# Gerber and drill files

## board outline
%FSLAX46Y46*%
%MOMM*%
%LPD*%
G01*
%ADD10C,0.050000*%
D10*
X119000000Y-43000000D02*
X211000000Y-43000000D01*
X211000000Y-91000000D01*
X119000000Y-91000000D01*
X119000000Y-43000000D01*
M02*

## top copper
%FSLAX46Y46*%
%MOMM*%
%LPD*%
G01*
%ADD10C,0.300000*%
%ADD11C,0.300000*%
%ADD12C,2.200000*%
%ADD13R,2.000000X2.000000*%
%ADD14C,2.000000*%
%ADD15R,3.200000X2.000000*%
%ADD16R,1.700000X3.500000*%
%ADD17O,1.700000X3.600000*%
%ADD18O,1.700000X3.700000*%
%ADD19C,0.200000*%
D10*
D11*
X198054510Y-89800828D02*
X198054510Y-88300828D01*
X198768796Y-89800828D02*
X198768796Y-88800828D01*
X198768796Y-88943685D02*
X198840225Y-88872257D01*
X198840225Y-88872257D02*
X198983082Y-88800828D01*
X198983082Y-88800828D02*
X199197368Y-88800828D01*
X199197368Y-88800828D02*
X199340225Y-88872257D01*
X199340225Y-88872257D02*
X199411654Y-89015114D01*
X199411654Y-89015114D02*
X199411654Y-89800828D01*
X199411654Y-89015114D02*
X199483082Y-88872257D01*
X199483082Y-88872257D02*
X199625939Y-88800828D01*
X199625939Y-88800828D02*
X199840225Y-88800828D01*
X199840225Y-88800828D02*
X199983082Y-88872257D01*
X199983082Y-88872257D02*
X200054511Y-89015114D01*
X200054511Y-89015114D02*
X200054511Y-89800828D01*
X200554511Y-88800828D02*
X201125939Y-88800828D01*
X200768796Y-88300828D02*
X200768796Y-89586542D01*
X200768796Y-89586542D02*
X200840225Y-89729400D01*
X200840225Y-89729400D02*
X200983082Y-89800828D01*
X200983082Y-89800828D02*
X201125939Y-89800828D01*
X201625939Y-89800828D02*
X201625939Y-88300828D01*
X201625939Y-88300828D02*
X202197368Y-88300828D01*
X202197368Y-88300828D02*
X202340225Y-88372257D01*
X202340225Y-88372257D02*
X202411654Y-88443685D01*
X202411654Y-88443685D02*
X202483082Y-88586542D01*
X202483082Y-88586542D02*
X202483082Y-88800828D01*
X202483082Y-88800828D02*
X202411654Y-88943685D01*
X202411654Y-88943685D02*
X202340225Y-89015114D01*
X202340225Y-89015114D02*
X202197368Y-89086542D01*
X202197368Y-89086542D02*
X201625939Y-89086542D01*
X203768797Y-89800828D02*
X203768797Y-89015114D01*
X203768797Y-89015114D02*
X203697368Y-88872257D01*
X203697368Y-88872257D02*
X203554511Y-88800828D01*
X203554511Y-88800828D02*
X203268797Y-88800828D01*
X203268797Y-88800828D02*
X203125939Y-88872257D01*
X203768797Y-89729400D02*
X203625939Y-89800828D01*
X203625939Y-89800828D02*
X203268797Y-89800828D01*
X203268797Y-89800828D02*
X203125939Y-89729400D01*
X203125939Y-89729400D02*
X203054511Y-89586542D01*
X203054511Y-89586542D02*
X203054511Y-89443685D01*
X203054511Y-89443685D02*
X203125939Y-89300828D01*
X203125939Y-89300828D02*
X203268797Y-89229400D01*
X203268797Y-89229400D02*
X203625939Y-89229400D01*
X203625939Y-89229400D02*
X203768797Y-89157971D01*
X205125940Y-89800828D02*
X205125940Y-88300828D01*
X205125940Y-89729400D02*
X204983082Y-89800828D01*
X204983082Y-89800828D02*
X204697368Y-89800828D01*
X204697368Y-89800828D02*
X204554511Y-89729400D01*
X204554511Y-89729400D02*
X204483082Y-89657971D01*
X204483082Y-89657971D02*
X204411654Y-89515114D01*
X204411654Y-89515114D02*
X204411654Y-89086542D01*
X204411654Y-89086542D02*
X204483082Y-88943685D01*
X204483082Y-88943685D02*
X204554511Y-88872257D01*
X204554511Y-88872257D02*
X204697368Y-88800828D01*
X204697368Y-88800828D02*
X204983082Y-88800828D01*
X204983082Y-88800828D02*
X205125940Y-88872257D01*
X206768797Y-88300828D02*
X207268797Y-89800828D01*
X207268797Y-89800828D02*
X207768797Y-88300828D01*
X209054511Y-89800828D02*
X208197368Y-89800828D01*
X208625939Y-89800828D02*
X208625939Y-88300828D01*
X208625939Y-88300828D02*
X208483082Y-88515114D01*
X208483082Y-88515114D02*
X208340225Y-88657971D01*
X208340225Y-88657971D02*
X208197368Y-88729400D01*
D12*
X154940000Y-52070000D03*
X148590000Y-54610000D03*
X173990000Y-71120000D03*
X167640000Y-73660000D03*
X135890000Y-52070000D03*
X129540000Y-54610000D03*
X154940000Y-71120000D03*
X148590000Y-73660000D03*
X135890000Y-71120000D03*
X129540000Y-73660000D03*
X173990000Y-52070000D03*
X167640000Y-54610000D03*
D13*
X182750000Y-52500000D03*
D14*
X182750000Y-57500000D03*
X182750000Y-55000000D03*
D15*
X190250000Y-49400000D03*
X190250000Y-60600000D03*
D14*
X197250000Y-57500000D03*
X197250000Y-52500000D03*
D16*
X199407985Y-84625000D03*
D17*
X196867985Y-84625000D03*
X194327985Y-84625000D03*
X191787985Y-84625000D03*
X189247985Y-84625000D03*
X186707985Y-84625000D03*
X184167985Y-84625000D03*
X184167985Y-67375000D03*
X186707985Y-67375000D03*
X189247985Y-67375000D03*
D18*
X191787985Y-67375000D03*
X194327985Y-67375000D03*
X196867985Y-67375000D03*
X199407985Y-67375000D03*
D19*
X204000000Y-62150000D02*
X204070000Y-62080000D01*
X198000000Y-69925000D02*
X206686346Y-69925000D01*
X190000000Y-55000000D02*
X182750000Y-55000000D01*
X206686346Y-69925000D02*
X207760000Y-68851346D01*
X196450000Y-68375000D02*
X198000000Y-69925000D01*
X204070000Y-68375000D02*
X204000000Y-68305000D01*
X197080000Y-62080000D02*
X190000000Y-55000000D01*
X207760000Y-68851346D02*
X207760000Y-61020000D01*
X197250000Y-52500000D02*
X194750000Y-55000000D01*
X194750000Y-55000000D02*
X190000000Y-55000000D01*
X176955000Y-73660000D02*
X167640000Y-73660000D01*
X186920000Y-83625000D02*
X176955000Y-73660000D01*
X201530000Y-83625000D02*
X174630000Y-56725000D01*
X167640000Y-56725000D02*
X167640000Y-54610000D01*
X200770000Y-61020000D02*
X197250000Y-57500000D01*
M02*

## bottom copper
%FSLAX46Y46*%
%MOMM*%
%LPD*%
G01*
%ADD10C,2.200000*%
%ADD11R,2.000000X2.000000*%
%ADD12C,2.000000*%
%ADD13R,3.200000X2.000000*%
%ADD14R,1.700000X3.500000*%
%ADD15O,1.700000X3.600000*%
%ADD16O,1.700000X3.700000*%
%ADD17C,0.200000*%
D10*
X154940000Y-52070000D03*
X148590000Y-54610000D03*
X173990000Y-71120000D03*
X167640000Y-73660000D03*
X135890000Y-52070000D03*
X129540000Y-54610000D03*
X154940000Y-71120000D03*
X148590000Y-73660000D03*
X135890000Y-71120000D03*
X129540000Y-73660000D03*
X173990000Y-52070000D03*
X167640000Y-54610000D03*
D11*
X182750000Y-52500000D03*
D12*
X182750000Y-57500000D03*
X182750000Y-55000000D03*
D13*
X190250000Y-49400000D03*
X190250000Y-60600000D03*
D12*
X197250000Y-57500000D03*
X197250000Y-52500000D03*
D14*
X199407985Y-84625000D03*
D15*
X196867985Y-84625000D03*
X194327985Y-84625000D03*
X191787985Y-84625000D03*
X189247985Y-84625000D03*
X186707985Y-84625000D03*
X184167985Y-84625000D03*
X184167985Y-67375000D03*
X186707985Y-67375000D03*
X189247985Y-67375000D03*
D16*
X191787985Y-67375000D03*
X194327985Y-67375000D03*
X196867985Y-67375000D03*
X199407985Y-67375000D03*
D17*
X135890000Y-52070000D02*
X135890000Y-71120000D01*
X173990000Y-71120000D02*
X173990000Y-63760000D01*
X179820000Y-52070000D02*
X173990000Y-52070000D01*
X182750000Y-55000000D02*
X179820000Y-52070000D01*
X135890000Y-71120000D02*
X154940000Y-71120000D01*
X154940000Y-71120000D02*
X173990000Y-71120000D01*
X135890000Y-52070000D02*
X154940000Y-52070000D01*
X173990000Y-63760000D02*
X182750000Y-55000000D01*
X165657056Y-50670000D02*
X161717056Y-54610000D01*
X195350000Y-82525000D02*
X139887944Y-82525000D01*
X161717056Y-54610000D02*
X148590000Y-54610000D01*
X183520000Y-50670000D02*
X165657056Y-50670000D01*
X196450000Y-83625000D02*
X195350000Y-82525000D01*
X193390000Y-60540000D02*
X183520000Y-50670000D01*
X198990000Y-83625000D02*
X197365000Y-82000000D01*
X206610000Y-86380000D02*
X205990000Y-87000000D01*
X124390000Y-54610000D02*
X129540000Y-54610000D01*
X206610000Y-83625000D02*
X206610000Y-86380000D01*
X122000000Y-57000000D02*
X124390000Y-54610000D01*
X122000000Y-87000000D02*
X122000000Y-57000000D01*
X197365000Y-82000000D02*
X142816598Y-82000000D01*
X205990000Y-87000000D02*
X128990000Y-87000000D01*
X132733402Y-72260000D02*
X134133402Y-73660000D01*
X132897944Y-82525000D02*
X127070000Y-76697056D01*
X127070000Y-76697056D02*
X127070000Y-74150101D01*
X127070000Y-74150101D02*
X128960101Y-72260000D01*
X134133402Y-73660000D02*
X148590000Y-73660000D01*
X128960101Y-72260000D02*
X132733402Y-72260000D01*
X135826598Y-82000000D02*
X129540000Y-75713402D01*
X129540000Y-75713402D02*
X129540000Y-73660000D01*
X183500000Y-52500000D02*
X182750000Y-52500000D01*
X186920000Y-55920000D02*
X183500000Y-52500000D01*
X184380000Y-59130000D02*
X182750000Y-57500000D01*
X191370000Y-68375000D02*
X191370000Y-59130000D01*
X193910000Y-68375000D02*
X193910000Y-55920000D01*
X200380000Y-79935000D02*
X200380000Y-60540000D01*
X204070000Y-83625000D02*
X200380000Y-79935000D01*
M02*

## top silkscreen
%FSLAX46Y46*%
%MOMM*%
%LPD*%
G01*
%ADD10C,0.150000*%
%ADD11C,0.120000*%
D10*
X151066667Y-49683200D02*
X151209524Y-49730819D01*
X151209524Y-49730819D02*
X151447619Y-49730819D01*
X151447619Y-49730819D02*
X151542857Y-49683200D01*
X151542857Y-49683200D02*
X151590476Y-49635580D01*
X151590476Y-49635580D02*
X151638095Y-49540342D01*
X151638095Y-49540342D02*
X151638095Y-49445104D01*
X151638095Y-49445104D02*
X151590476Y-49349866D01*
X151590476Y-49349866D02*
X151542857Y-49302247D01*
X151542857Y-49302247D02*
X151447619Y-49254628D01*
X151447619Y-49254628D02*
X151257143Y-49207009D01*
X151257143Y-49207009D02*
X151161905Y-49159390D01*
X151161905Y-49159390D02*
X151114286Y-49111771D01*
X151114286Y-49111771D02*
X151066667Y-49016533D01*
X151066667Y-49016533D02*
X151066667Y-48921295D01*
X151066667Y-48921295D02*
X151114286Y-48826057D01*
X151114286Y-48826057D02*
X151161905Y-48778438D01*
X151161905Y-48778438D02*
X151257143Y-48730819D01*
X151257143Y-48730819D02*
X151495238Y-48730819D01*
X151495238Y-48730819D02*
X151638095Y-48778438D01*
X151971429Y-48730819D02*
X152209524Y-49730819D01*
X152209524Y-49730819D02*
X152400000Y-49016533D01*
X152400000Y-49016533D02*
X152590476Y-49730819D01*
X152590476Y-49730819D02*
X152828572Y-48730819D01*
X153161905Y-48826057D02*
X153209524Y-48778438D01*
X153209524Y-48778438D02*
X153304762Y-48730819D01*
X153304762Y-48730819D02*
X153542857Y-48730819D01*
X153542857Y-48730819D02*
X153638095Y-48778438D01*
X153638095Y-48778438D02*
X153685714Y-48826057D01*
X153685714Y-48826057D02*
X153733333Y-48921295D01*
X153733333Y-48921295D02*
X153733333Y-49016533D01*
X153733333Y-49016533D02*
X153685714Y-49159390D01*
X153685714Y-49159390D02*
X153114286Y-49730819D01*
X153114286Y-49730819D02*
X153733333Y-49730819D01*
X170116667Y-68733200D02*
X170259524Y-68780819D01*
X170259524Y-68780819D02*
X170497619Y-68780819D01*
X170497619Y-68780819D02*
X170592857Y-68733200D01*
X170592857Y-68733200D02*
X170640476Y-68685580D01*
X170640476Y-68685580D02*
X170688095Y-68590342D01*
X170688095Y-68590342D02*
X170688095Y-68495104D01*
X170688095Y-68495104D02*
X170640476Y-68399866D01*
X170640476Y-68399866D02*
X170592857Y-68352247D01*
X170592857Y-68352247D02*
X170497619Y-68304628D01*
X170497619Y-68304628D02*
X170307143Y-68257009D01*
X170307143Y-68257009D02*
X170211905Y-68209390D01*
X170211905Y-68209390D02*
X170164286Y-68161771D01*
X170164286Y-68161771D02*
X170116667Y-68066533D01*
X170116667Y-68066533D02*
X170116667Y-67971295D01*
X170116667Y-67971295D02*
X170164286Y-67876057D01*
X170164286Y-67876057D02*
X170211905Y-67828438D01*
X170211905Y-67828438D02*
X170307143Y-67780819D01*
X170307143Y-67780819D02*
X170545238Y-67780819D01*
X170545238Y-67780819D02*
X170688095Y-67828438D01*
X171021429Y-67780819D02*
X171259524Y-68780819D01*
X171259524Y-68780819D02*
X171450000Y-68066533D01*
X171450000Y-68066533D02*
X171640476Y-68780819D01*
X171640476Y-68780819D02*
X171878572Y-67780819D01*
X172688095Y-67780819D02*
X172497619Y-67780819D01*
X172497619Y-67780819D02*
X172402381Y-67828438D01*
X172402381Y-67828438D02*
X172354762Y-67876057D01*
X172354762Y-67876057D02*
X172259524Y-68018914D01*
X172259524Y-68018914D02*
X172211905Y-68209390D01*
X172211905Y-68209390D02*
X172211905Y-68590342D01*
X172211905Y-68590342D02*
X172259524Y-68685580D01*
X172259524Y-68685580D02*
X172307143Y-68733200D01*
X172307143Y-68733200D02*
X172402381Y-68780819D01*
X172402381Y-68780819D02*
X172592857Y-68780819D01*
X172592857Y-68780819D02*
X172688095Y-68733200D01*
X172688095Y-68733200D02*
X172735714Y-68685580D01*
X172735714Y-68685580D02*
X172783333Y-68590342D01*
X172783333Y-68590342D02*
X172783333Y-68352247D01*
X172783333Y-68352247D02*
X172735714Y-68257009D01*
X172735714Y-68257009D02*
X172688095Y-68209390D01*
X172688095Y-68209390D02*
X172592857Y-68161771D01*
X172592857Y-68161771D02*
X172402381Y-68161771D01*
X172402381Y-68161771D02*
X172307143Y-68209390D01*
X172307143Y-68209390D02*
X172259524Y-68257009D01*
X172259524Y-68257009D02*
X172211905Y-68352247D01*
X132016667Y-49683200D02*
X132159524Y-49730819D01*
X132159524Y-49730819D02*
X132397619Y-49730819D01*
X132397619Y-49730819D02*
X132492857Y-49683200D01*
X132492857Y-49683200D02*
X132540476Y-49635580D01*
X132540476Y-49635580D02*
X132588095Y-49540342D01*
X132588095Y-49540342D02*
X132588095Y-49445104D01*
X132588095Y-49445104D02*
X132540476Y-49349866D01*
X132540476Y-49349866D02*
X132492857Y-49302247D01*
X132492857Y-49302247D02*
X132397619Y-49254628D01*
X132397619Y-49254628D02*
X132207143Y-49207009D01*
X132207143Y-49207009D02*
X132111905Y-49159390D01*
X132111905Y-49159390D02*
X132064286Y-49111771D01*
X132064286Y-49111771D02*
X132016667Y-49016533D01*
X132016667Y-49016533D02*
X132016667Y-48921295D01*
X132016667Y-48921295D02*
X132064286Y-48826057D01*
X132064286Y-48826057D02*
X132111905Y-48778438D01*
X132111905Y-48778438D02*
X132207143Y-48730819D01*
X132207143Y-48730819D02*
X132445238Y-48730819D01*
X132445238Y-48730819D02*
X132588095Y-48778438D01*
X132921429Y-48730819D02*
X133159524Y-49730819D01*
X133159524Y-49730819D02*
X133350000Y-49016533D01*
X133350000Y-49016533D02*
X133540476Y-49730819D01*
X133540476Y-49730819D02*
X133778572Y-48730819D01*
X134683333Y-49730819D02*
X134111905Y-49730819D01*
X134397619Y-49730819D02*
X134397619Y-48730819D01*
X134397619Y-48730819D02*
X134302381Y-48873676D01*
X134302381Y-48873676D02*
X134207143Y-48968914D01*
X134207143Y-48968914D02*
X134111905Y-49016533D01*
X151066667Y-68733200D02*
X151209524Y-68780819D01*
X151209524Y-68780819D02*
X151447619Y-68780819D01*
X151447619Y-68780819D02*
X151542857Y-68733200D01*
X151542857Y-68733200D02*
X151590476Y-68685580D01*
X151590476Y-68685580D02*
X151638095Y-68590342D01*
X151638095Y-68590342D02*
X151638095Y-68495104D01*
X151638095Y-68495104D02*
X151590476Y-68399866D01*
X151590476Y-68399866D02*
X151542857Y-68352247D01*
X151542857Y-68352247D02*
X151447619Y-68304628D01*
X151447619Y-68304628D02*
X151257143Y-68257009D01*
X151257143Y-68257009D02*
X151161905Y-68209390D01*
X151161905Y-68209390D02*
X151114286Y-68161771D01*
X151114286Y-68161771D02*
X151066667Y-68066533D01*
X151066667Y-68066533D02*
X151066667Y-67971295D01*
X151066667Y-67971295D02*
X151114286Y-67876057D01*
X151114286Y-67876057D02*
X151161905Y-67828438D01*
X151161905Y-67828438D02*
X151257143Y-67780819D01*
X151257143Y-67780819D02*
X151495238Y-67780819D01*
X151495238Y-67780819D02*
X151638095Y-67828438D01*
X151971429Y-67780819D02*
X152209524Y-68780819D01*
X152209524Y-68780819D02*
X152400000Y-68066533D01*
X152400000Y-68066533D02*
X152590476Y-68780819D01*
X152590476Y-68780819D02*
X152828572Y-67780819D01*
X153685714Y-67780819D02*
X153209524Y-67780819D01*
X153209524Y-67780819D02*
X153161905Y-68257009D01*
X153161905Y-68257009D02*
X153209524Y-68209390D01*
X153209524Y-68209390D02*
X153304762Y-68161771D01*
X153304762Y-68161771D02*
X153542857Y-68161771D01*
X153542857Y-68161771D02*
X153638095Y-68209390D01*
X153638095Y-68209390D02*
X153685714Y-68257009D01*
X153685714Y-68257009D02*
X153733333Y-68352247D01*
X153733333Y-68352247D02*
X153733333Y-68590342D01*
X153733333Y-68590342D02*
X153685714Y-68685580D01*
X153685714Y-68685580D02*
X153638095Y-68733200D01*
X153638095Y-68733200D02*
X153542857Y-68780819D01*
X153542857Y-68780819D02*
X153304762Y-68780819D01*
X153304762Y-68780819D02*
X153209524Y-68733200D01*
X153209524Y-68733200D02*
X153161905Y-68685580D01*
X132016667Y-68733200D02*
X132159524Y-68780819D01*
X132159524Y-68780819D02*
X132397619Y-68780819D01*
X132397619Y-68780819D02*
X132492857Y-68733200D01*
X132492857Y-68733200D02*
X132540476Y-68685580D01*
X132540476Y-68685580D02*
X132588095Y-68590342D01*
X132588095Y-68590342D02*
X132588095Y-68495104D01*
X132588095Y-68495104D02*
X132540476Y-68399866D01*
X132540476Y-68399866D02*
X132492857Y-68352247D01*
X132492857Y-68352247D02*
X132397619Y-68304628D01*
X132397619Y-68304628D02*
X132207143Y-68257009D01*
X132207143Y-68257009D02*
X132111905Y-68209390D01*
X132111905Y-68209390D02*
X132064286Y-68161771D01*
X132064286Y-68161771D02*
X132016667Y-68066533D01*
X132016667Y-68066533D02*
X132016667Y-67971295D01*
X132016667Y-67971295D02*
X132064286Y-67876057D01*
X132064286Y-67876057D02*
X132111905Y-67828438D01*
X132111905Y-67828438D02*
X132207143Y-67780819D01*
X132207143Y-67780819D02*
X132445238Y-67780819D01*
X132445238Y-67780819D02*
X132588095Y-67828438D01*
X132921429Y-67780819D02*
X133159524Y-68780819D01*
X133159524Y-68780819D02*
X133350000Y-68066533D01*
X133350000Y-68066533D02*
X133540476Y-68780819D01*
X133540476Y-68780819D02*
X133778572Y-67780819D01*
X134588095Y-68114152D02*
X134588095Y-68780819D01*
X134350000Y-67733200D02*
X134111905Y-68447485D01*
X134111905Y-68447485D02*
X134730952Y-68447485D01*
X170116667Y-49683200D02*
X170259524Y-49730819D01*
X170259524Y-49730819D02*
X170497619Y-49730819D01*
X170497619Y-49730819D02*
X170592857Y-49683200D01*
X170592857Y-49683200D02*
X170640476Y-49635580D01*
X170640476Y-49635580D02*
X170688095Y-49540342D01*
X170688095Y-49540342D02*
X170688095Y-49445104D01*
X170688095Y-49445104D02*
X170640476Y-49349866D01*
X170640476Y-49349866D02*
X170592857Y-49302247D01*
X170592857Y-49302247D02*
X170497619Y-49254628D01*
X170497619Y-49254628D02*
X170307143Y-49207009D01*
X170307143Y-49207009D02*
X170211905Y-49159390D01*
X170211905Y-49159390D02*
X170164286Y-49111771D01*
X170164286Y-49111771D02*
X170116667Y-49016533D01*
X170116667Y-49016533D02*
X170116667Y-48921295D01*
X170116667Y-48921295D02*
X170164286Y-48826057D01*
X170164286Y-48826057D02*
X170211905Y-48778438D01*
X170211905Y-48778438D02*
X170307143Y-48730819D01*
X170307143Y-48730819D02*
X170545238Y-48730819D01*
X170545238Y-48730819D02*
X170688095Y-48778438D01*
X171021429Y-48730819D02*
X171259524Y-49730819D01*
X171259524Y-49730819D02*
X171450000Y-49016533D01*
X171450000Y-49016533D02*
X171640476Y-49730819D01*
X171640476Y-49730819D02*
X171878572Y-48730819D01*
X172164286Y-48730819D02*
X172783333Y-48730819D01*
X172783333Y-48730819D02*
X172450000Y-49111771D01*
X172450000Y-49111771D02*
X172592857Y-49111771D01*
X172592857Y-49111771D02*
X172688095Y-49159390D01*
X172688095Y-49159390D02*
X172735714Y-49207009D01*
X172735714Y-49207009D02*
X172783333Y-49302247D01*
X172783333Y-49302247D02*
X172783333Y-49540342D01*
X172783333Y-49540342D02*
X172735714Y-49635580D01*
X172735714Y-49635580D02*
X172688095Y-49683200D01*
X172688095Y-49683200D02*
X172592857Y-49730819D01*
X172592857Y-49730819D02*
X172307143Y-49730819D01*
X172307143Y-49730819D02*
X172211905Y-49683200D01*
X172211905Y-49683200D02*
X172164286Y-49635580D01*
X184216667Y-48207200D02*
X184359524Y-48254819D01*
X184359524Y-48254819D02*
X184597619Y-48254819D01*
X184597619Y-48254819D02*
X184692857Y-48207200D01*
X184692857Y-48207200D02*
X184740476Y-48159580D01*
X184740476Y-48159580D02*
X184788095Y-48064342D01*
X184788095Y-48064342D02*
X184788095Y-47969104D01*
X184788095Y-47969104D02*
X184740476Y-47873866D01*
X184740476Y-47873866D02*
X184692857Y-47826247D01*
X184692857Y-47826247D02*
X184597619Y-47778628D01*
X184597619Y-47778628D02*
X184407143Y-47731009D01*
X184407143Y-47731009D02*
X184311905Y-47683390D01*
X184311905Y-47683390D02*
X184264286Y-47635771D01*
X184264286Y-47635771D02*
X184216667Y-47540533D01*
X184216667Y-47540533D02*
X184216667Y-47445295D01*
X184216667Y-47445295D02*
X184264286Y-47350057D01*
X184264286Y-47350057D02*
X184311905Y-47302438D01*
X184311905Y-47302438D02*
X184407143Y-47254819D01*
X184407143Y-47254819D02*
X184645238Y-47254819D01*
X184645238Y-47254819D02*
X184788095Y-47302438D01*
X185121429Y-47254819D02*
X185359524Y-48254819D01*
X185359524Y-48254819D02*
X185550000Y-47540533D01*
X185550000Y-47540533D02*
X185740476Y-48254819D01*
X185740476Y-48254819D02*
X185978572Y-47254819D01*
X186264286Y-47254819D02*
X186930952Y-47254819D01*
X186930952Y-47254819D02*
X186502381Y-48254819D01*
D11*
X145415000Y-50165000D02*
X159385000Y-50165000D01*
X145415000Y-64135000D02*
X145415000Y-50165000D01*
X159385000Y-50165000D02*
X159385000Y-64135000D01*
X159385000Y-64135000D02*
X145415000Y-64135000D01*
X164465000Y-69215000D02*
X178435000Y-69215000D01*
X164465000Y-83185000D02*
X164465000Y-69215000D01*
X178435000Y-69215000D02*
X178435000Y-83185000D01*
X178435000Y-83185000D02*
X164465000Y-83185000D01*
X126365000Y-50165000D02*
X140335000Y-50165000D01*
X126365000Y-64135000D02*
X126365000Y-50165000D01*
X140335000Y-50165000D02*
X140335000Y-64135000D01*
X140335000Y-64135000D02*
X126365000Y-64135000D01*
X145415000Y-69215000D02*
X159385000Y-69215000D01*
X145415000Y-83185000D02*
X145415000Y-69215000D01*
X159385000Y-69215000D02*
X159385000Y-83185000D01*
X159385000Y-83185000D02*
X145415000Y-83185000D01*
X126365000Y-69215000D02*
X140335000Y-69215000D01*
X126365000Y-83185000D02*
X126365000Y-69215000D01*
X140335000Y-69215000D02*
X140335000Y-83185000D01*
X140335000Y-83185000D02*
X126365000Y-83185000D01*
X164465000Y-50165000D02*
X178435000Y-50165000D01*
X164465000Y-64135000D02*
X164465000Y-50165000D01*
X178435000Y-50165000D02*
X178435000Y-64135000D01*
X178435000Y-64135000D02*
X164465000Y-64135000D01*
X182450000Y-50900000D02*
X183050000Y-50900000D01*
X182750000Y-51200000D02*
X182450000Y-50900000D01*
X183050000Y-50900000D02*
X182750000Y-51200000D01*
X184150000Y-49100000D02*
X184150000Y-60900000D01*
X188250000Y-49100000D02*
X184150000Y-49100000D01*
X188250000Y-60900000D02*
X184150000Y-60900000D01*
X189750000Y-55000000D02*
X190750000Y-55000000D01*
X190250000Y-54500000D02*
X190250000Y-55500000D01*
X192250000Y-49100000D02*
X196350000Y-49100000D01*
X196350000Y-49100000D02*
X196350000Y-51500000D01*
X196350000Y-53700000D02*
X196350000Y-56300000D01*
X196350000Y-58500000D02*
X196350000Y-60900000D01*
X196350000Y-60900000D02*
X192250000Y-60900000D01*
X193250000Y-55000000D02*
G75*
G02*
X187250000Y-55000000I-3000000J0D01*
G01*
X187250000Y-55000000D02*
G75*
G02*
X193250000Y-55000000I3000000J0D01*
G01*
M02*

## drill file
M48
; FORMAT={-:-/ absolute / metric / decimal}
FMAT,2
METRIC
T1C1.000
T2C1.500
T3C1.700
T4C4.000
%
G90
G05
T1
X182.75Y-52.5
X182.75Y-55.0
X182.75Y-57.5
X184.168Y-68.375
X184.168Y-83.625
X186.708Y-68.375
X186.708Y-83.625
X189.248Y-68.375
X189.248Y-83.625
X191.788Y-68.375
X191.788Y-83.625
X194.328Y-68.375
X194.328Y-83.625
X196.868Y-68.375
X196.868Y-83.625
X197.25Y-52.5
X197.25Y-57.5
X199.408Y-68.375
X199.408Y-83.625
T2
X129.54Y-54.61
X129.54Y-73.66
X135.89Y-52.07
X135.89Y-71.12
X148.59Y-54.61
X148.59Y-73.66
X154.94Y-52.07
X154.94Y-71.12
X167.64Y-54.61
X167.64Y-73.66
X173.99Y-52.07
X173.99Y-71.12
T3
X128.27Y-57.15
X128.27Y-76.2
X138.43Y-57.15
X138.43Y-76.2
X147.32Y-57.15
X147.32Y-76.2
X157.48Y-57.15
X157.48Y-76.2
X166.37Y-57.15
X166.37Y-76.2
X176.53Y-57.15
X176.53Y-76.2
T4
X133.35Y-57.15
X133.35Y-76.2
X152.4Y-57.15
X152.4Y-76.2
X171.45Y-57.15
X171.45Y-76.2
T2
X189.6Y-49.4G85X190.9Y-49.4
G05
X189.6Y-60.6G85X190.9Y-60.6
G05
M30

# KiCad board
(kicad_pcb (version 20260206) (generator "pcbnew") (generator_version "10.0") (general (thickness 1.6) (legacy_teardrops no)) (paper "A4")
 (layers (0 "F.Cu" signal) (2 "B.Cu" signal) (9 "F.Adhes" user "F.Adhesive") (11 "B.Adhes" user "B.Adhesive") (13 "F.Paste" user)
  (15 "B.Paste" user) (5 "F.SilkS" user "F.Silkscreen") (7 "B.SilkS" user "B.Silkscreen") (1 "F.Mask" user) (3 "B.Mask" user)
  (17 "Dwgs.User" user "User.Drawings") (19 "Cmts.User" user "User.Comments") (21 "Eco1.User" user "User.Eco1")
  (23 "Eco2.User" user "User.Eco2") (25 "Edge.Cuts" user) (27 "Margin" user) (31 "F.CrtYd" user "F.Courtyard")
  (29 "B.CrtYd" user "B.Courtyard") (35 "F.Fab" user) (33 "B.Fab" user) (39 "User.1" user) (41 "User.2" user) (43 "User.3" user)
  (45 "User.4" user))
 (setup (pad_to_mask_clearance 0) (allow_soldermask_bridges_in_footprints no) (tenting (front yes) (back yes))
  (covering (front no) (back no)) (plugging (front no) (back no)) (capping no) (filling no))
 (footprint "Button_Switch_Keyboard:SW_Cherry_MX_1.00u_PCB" (layer "F.Cu") (at 154.94 52.07)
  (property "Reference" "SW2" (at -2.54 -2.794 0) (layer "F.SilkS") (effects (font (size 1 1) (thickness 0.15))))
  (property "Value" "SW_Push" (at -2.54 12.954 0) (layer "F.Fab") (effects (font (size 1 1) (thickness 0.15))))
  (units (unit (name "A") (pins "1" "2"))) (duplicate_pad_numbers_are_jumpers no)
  (fp_line (start -9.525 -1.905) (end 4.445 -1.905) (stroke (width 0.12) (type solid)) (layer "F.SilkS"))
  (fp_line (start -9.525 12.065) (end -9.525 -1.905) (stroke (width 0.12) (type solid)) (layer "F.SilkS"))
  (fp_line (start 4.445 -1.905) (end 4.445 12.065) (stroke (width 0.12) (type solid)) (layer "F.SilkS"))
  (fp_line (start 4.445 12.065) (end -9.525 12.065) (stroke (width 0.12) (type solid)) (layer "F.SilkS"))
  (pad "" np_thru_hole circle (at -7.62 5.08) (size 1.7 1.7) (drill 1.7) (layers "*.Cu" "*.Mask"))
  (pad "" np_thru_hole circle (at -2.54 5.08) (size 4 4) (drill 4) (layers "*.Cu" "*.Mask"))
  (pad "" np_thru_hole circle (at 2.54 5.08) (size 1.7 1.7) (drill 1.7) (layers "*.Cu" "*.Mask"))
  (pad "1" thru_hole circle (at 0 0) (size 2.2 2.2) (drill 1.5) (layers "*.Cu" "*.Mask") (remove_unused_layers no) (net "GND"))
  (pad "2" thru_hole circle (at -6.35 2.54) (size 2.2 2.2) (drill 1.5) (layers "*.Cu" "*.Mask") (remove_unused_layers no)
   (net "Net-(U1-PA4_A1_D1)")))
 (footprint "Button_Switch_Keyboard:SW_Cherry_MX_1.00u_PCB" (layer "F.Cu") (at 173.99 71.12)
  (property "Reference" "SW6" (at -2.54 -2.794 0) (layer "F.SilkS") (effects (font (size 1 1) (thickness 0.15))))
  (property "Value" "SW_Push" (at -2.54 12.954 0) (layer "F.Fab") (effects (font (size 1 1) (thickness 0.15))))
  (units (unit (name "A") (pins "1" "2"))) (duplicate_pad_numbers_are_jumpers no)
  (fp_line (start -9.525 -1.905) (end 4.445 -1.905) (stroke (width 0.12) (type solid)) (layer "F.SilkS"))
  (fp_line (start -9.525 12.065) (end -9.525 -1.905) (stroke (width 0.12) (type solid)) (layer "F.SilkS"))
  (fp_line (start 4.445 -1.905) (end 4.445 12.065) (stroke (width 0.12) (type solid)) (layer "F.SilkS"))
  (fp_line (start 4.445 12.065) (end -9.525 12.065) (stroke (width 0.12) (type solid)) (layer "F.SilkS"))
  (pad "" np_thru_hole circle (at -7.62 5.08) (size 1.7 1.7) (drill 1.7) (layers "*.Cu" "*.Mask"))
  (pad "" np_thru_hole circle (at -2.54 5.08) (size 4 4) (drill 4) (layers "*.Cu" "*.Mask"))
  (pad "" np_thru_hole circle (at 2.54 5.08) (size 1.7 1.7) (drill 1.7) (layers "*.Cu" "*.Mask"))
  (pad "1" thru_hole circle (at 0 0) (size 2.2 2.2) (drill 1.5) (layers "*.Cu" "*.Mask") (remove_unused_layers no) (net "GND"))
  (pad "2" thru_hole circle (at -6.35 2.54) (size 2.2 2.2) (drill 1.5) (layers "*.Cu" "*.Mask") (remove_unused_layers no)
   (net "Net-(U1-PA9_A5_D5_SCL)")))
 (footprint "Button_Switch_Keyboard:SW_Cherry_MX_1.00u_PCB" (layer "F.Cu") (at 135.89 52.07)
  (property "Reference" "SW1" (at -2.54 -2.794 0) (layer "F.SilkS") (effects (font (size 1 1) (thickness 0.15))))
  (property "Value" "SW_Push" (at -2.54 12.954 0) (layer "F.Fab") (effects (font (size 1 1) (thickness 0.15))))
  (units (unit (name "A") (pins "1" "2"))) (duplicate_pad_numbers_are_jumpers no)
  (fp_line (start -9.525 -1.905) (end 4.445 -1.905) (stroke (width 0.12) (type solid)) (layer "F.SilkS"))
  (fp_line (start -9.525 12.065) (end -9.525 -1.905) (stroke (width 0.12) (type solid)) (layer "F.SilkS"))
  (fp_line (start 4.445 -1.905) (end 4.445 12.065) (stroke (width 0.12) (type solid)) (layer "F.SilkS"))
  (fp_line (start 4.445 12.065) (end -9.525 12.065) (stroke (width 0.12) (type solid)) (layer "F.SilkS"))
  (pad "" np_thru_hole circle (at -7.62 5.08) (size 1.7 1.7) (drill 1.7) (layers "*.Cu" "*.Mask"))
  (pad "" np_thru_hole circle (at -2.54 5.08) (size 4 4) (drill 4) (layers "*.Cu" "*.Mask"))
  (pad "" np_thru_hole circle (at 2.54 5.08) (size 1.7 1.7) (drill 1.7) (layers "*.Cu" "*.Mask"))
  (pad "1" thru_hole circle (at 0 0) (size 2.2 2.2) (drill 1.5) (layers "*.Cu" "*.Mask") (remove_unused_layers no) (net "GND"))
  (pad "2" thru_hole circle (at -6.35 2.54) (size 2.2 2.2) (drill 1.5) (layers "*.Cu" "*.Mask") (remove_unused_layers no)
   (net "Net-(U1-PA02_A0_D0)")))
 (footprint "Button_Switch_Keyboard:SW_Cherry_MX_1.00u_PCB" (layer "F.Cu") (at 154.94 71.12)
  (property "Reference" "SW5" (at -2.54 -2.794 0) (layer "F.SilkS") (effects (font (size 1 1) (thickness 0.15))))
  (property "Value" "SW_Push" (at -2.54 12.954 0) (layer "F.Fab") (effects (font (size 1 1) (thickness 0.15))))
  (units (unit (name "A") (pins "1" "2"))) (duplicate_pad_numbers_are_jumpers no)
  (fp_line (start -9.525 -1.905) (end 4.445 -1.905) (stroke (width 0.12) (type solid)) (layer "F.SilkS"))
  (fp_line (start -9.525 12.065) (end -9.525 -1.905) (stroke (width 0.12) (type solid)) (layer "F.SilkS"))
  (fp_line (start 4.445 -1.905) (end 4.445 12.065) (stroke (width 0.12) (type solid)) (layer "F.SilkS"))
  (fp_line (start 4.445 12.065) (end -9.525 12.065) (stroke (width 0.12) (type solid)) (layer "F.SilkS"))
  (pad "" np_thru_hole circle (at -7.62 5.08) (size 1.7 1.7) (drill 1.7) (layers "*.Cu" "*.Mask"))
  (pad "" np_thru_hole circle (at -2.54 5.08) (size 4 4) (drill 4) (layers "*.Cu" "*.Mask"))
  (pad "" np_thru_hole circle (at 2.54 5.08) (size 1.7 1.7) (drill 1.7) (layers "*.Cu" "*.Mask"))
  (pad "1" thru_hole circle (at 0 0) (size 2.2 2.2) (drill 1.5) (layers "*.Cu" "*.Mask") (remove_unused_layers no) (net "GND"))
  (pad "2" thru_hole circle (at -6.35 2.54) (size 2.2 2.2) (drill 1.5) (layers "*.Cu" "*.Mask") (remove_unused_layers no)
   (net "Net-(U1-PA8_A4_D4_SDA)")))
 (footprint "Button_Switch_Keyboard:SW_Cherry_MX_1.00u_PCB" (layer "F.Cu") (at 135.89 71.12)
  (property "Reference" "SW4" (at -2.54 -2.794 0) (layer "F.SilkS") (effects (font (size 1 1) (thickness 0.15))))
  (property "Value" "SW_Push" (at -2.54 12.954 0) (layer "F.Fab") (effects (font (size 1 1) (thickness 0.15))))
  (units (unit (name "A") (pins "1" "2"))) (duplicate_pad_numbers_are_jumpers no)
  (fp_line (start -9.525 -1.905) (end 4.445 -1.905) (stroke (width 0.12) (type solid)) (layer "F.SilkS"))
  (fp_line (start -9.525 12.065) (end -9.525 -1.905) (stroke (width 0.12) (type solid)) (layer "F.SilkS"))
  (fp_line (start 4.445 -1.905) (end 4.445 12.065) (stroke (width 0.12) (type solid)) (layer "F.SilkS"))
  (fp_line (start 4.445 12.065) (end -9.525 12.065) (stroke (width 0.12) (type solid)) (layer "F.SilkS"))
  (pad "" np_thru_hole circle (at -7.62 5.08) (size 1.7 1.7) (drill 1.7) (layers "*.Cu" "*.Mask"))
  (pad "" np_thru_hole circle (at -2.54 5.08) (size 4 4) (drill 4) (layers "*.Cu" "*.Mask"))
  (pad "" np_thru_hole circle (at 2.54 5.08) (size 1.7 1.7) (drill 1.7) (layers "*.Cu" "*.Mask"))
  (pad "1" thru_hole circle (at 0 0) (size 2.2 2.2) (drill 1.5) (layers "*.Cu" "*.Mask") (remove_unused_layers no) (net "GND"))
  (pad "2" thru_hole circle (at -6.35 2.54) (size 2.2 2.2) (drill 1.5) (layers "*.Cu" "*.Mask") (remove_unused_layers no)
   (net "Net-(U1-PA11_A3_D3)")))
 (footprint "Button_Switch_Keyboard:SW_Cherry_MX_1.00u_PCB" (layer "F.Cu") (at 173.99 52.07)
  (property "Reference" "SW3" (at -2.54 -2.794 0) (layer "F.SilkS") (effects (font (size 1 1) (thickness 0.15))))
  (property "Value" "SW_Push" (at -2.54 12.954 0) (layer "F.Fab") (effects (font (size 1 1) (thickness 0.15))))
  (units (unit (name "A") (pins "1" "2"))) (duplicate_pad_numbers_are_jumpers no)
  (fp_line (start -9.525 -1.905) (end 4.445 -1.905) (stroke (width 0.12) (type solid)) (layer "F.SilkS"))
  (fp_line (start -9.525 12.065) (end -9.525 -1.905) (stroke (width 0.12) (type solid)) (layer "F.SilkS"))
  (fp_line (start 4.445 -1.905) (end 4.445 12.065) (stroke (width 0.12) (type solid)) (layer "F.SilkS"))
  (fp_line (start 4.445 12.065) (end -9.525 12.065) (stroke (width 0.12) (type solid)) (layer "F.SilkS"))
  (pad "" np_thru_hole circle (at -7.62 5.08) (size 1.7 1.7) (drill 1.7) (layers "*.Cu" "*.Mask"))
  (pad "" np_thru_hole circle (at -2.54 5.08) (size 4 4) (drill 4) (layers "*.Cu" "*.Mask"))
  (pad "" np_thru_hole circle (at 2.54 5.08) (size 1.7 1.7) (drill 1.7) (layers "*.Cu" "*.Mask"))
  (pad "1" thru_hole circle (at 0 0) (size 2.2 2.2) (drill 1.5) (layers "*.Cu" "*.Mask") (remove_unused_layers no) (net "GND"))
  (pad "2" thru_hole circle (at -6.35 2.54) (size 2.2 2.2) (drill 1.5) (layers "*.Cu" "*.Mask") (remove_unused_layers no)
   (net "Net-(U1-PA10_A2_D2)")))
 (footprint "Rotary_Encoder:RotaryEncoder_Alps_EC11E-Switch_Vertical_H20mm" (layer "F.Cu") (at 182.75 52.5)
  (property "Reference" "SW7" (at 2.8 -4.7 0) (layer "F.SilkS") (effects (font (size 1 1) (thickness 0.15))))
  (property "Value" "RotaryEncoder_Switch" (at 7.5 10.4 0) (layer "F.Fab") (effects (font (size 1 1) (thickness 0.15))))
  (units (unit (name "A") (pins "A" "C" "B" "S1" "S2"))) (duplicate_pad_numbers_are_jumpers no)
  (fp_line (start -0.3 -1.6) (end 0.3 -1.6) (stroke (width 0.12) (type solid)) (layer "F.SilkS"))
  (fp_line (start 0 -1.3) (end -0.3 -1.6) (stroke (width 0.12) (type solid)) (layer "F.SilkS"))
  (fp_line (start 0.3 -1.6) (end 0 -1.3) (stroke (width 0.12) (type solid)) (layer "F.SilkS"))
  (fp_line (start 1.4 -3.4) (end 1.4 8.4) (stroke (width 0.12) (type solid)) (layer "F.SilkS"))
  (fp_line (start 5.5 -3.4) (end 1.4 -3.4) (stroke (width 0.12) (type solid)) (layer "F.SilkS"))
  (fp_line (start 5.5 8.4) (end 1.4 8.4) (stroke (width 0.12) (type solid)) (layer "F.SilkS"))
  (fp_line (start 7 2.5) (end 8 2.5) (stroke (width 0.12) (type solid)) (layer "F.SilkS"))
  (fp_line (start 7.5 2) (end 7.5 3) (stroke (width 0.12) (type solid)) (layer "F.SilkS"))
  (fp_line (start 9.5 -3.4) (end 13.6 -3.4) (stroke (width 0.12) (type solid)) (layer "F.SilkS"))
  (fp_line (start 13.6 -3.4) (end 13.6 -1) (stroke (width 0.12) (type solid)) (layer "F.SilkS"))
  (fp_line (start 13.6 1.2) (end 13.6 3.8) (stroke (width 0.12) (type solid)) (layer "F.SilkS"))
  (fp_line (start 13.6 6) (end 13.6 8.4) (stroke (width 0.12) (type solid)) (layer "F.SilkS"))
  (fp_line (start 13.6 8.4) (end 9.5 8.4) (stroke (width 0.12) (type solid)) (layer "F.SilkS"))
  (fp_circle (center 7.5 2.5) (end 10.5 2.5) (stroke (width 0.12) (type solid)) (fill no) (layer "F.SilkS"))
  (pad "A" thru_hole rect (at 0 0) (size 2 2) (drill 1) (layers "*.Cu" "*.Mask") (remove_unused_layers no) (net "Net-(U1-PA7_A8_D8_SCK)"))
  (pad "B" thru_hole circle (at 0 5) (size 2 2) (drill 1) (layers "*.Cu" "*.Mask") (remove_unused_layers no) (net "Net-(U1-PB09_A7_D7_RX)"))
  (pad "C" thru_hole circle (at 0 2.5) (size 2 2) (drill 1) (layers "*.Cu" "*.Mask") (remove_unused_layers no) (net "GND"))
  (pad "MP" thru_hole rect (at 7.5 -3.1) (size 3.2 2) (drill oval 2.8 1.5) (layers "*.Cu" "*.Mask") (remove_unused_layers no))
  (pad "MP" thru_hole rect (at 7.5 8.1) (size 3.2 2) (drill oval 2.8 1.5) (layers "*.Cu" "*.Mask") (remove_unused_layers no))
  (pad "S1" thru_hole circle (at 14.5 5) (size 2 2) (drill 1) (layers "*.Cu" "*.Mask") (remove_unused_layers no)
   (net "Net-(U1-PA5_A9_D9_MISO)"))
  (pad "S2" thru_hole circle (at 14.5 0) (size 2 2) (drill 1) (layers "*.Cu" "*.Mask") (remove_unused_layers no) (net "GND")))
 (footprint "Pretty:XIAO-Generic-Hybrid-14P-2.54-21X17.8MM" (layer "B.Cu") (at 191.787985 76 90)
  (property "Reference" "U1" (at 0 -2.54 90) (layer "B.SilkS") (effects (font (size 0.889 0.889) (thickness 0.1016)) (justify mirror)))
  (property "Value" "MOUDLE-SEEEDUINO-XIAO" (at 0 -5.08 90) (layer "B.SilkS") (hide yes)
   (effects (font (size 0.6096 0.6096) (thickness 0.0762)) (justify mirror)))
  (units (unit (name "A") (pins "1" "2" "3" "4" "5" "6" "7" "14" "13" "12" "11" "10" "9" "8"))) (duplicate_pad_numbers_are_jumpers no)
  (pad "1" thru_hole rect (at -7.625 7.62 90) (size 3.5 1.7) (drill 1 (offset -1 0)) (layers "*.Cu" "*.Mask") (remove_unused_layers no)
   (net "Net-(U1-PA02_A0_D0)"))
  (pad "2" thru_hole oval (at -7.625 5.08 90) (size 3.6 1.7) (drill 1 (offset -1 0)) (layers "*.Cu" "*.Mask") (remove_unused_layers no)
   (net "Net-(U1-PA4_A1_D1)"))
  (pad "3" thru_hole oval (at -7.625 2.54 90) (size 3.6 1.7) (drill 1 (offset -1 0)) (layers "*.Cu" "*.Mask") (remove_unused_layers no)
   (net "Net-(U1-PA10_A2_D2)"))
  (pad "4" thru_hole oval (at -7.625 0 90) (size 3.6 1.7) (drill 1 (offset -1 0)) (layers "*.Cu" "*.Mask") (remove_unused_layers no)
   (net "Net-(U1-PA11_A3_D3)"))
  (pad "5" thru_hole oval (at -7.625 -2.54 90) (size 3.6 1.7) (drill 1 (offset -1 0)) (layers "*.Cu" "*.Mask") (remove_unused_layers no)
   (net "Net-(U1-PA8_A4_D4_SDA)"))
  (pad "6" thru_hole oval (at -7.625 -5.08 270) (size 3.6 1.7) (drill 1 (offset 1 0)) (layers "*.Cu" "*.Mask") (remove_unused_layers no)
   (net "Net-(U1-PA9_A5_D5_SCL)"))
  (pad "7" thru_hole oval (at -7.625 -7.62 90) (size 3.6 1.7) (drill 1 (offset -1 0)) (layers "*.Cu" "*.Mask") (remove_unused_layers no)
   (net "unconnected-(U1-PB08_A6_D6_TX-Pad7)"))
  (pad "8" thru_hole oval (at 7.625 -7.62 90) (size 3.6 1.7) (drill 1 (offset 1 0)) (layers "*.Cu" "*.Mask") (remove_unused_layers no)
   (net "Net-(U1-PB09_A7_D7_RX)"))
  (pad "9" thru_hole oval (at 7.625 -5.08 90) (size 3.6 1.7) (drill 1 (offset 1 0)) (layers "*.Cu" "*.Mask") (remove_unused_layers no)
   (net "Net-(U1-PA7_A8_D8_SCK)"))
  (pad "10" thru_hole oval (at 7.625 -2.54 90) (size 3.6 1.7) (drill 1 (offset 1 0)) (layers "*.Cu" "*.Mask") (remove_unused_layers no)
   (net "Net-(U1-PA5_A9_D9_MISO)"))
  (pad "11" thru_hole oval (at 7.625 0 90) (size 3.7 1.7) (drill 1 (offset 1 0)) (layers "*.Cu" "*.Mask") (remove_unused_layers no)
   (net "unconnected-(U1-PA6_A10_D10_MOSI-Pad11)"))
  (pad "12" thru_hole oval (at 7.625 2.54 90) (size 3.7 1.7) (drill 1 (offset 1 0)) (layers "*.Cu" "*.Mask") (remove_unused_layers no)
   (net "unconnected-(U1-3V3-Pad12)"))
  (pad "13" thru_hole oval (at 7.625 5.08 90) (size 3.7 1.7) (drill 1 (offset 1 0)) (layers "*.Cu" "*.Mask") (remove_unused_layers no)
   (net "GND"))
  (pad "14" thru_hole oval (at 7.625 7.62 90) (size 3.7 1.7) (drill 1 (offset 1 0)) (layers "*.Cu" "*.Mask") (remove_unused_layers no)
   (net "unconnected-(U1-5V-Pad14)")))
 (gr_rect (start 119 43) (end 211 91) (stroke (width 0.05) (type default)) (fill no) (layer "Edge.Cuts"))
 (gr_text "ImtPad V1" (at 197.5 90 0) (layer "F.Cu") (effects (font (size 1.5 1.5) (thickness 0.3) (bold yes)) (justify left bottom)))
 (segment (start 204 62.15) (end 204.07 62.08) (width 0.2) (layer "F.Cu") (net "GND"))
 (segment (start 198 69.925) (end 206.686346 69.925) (width 0.2) (layer "F.Cu") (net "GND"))
 (segment (start 190 55) (end 182.75 55) (width 0.2) (layer "F.Cu") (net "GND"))
 (segment (start 206.686346 69.925) (end 207.76 68.851346) (width 0.2) (layer "F.Cu") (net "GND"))
 (segment (start 196.45 68.375) (end 198 69.925) (width 0.2) (layer "F.Cu") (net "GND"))
 (segment (start 204.07 68.375) (end 204 68.305) (width 0.2) (layer "F.Cu") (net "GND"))
 (segment (start 197.08 62.08) (end 190 55) (width 0.2) (layer "F.Cu") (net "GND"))
 (segment (start 207.76 68.851346) (end 207.76 61.02) (width 0.2) (layer "F.Cu") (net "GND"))
 (segment (start 197.25 52.5) (end 194.75 55) (width 0.2) (layer "F.Cu") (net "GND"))
 (segment (start 194.75 55) (end 190 55) (width 0.2) (layer "F.Cu") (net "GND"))
 (segment (start 135.89 52.07) (end 135.89 71.12) (width 0.2) (layer "B.Cu") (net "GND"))
 (segment (start 173.99 71.12) (end 173.99 63.76) (width 0.2) (layer "B.Cu") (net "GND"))
 (segment (start 179.82 52.07) (end 173.99 52.07) (width 0.2) (layer "B.Cu") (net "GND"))
 (segment (start 182.75 55) (end 179.82 52.07) (width 0.2) (layer "B.Cu") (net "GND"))
 (segment (start 135.89 71.12) (end 154.94 71.12) (width 0.2) (layer "B.Cu") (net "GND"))
 (segment (start 154.94 71.12) (end 173.99 71.12) (width 0.2) (layer "B.Cu") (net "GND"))
 (segment (start 135.89 52.07) (end 154.94 52.07) (width 0.2) (layer "B.Cu") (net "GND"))
 (segment (start 173.99 63.76) (end 182.75 55) (width 0.2) (layer "B.Cu") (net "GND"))
 (segment (start 165.657056 50.67) (end 161.717056 54.61) (width 0.2) (layer "B.Cu") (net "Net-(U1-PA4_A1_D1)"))
 (segment (start 195.35 82.525) (end 139.887944 82.525) (width 0.2) (layer "B.Cu") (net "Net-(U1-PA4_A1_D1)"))
 (segment (start 161.717056 54.61) (end 148.59 54.61) (width 0.2) (layer "B.Cu") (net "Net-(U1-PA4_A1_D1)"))
 (segment (start 183.52 50.67) (end 165.657056 50.67) (width 0.2) (layer "B.Cu") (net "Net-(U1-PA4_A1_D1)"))
 (segment (start 196.45 83.625) (end 195.35 82.525) (width 0.2) (layer "B.Cu") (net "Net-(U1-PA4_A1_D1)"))
 (segment (start 193.39 60.54) (end 183.52 50.67) (width 0.2) (layer "B.Cu") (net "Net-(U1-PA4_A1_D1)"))
 (segment (start 176.955 73.66) (end 167.64 73.66) (width 0.2) (layer "F.Cu") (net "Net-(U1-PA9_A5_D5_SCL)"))
 (segment (start 186.92 83.625) (end 176.955 73.66) (width 0.2) (layer "F.Cu") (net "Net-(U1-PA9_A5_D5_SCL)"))
 (segment (start 198.99 83.625) (end 197.365 82) (width 0.2) (layer "B.Cu") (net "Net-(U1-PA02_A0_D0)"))
 (segment (start 206.61 86.38) (end 205.99 87) (width 0.2) (layer "B.Cu") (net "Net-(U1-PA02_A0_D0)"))
 (segment (start 124.39 54.61) (end 129.54 54.61) (width 0.2) (layer "B.Cu") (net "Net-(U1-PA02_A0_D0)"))
 (segment (start 206.61 83.625) (end 206.61 86.38) (width 0.2) (layer "B.Cu") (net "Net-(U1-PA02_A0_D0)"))
 (segment (start 122 57) (end 124.39 54.61) (width 0.2) (layer "B.Cu") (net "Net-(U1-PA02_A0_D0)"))
 (segment (start 122 87) (end 122 57) (width 0.2) (layer "B.Cu") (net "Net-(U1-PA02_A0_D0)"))
 (segment (start 197.365 82) (end 142.816598 82) (width 0.2) (layer "B.Cu") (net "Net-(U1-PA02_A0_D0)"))
 (segment (start 205.99 87) (end 128.99 87) (width 0.2) (layer "B.Cu") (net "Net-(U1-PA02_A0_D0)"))
 (segment (start 132.733402 72.26) (end 134.133402 73.66) (width 0.2) (layer "B.Cu") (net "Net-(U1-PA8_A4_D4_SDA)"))
 (segment (start 132.897944 82.525) (end 127.07 76.697056) (width 0.2) (layer "B.Cu") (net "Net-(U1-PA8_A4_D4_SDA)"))
 (segment (start 127.07 76.697056) (end 127.07 74.150101) (width 0.2) (layer "B.Cu") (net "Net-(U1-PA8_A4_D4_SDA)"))
 (segment (start 127.07 74.150101) (end 128.960101 72.26) (width 0.2) (layer "B.Cu") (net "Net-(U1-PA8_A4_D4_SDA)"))
 (segment (start 134.133402 73.66) (end 148.59 73.66) (width 0.2) (layer "B.Cu") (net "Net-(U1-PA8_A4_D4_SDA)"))
 (segment (start 128.960101 72.26) (end 132.733402 72.26) (width 0.2) (layer "B.Cu") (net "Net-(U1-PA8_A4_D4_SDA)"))
 (segment (start 135.826598 82) (end 129.54 75.713402) (width 0.2) (layer "B.Cu") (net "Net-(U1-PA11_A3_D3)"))
 (segment (start 129.54 75.713402) (end 129.54 73.66) (width 0.2) (layer "B.Cu") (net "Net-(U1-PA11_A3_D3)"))
 (segment (start 201.53 83.625) (end 174.63 56.725) (width 0.2) (layer "F.Cu") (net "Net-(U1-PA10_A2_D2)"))
 (segment (start 167.64 56.725) (end 167.64 54.61) (width 0.2) (layer "F.Cu") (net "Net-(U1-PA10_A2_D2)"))
 (segment (start 183.5 52.5) (end 182.75 52.5) (width 0.2) (layer "B.Cu") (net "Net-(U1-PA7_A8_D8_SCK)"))
 (segment (start 186.92 55.92) (end 183.5 52.5) (width 0.2) (layer "B.Cu") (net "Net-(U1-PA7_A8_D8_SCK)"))
 (segment (start 184.38 59.13) (end 182.75 57.5) (width 0.2) (layer "B.Cu") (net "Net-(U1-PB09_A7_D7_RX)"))
 (segment (start 200.77 61.02) (end 197.25 57.5) (width 0.2) (layer "F.Cu") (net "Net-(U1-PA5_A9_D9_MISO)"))
 (segment (start 191.37 68.375) (end 191.37 59.13) (width 0.2) (layer "B.Cu") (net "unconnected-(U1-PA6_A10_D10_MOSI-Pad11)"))
 (segment (start 193.91 68.375) (end 193.91 55.92) (width 0.2) (layer "B.Cu") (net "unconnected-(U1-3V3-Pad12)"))
 (segment (start 200.38 79.935) (end 200.38 60.54) (width 0.2) (layer "B.Cu") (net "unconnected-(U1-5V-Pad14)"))
 (segment (start 204.07 83.625) (end 200.38 79.935) (width 0.2) (layer "B.Cu") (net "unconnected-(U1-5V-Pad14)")))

